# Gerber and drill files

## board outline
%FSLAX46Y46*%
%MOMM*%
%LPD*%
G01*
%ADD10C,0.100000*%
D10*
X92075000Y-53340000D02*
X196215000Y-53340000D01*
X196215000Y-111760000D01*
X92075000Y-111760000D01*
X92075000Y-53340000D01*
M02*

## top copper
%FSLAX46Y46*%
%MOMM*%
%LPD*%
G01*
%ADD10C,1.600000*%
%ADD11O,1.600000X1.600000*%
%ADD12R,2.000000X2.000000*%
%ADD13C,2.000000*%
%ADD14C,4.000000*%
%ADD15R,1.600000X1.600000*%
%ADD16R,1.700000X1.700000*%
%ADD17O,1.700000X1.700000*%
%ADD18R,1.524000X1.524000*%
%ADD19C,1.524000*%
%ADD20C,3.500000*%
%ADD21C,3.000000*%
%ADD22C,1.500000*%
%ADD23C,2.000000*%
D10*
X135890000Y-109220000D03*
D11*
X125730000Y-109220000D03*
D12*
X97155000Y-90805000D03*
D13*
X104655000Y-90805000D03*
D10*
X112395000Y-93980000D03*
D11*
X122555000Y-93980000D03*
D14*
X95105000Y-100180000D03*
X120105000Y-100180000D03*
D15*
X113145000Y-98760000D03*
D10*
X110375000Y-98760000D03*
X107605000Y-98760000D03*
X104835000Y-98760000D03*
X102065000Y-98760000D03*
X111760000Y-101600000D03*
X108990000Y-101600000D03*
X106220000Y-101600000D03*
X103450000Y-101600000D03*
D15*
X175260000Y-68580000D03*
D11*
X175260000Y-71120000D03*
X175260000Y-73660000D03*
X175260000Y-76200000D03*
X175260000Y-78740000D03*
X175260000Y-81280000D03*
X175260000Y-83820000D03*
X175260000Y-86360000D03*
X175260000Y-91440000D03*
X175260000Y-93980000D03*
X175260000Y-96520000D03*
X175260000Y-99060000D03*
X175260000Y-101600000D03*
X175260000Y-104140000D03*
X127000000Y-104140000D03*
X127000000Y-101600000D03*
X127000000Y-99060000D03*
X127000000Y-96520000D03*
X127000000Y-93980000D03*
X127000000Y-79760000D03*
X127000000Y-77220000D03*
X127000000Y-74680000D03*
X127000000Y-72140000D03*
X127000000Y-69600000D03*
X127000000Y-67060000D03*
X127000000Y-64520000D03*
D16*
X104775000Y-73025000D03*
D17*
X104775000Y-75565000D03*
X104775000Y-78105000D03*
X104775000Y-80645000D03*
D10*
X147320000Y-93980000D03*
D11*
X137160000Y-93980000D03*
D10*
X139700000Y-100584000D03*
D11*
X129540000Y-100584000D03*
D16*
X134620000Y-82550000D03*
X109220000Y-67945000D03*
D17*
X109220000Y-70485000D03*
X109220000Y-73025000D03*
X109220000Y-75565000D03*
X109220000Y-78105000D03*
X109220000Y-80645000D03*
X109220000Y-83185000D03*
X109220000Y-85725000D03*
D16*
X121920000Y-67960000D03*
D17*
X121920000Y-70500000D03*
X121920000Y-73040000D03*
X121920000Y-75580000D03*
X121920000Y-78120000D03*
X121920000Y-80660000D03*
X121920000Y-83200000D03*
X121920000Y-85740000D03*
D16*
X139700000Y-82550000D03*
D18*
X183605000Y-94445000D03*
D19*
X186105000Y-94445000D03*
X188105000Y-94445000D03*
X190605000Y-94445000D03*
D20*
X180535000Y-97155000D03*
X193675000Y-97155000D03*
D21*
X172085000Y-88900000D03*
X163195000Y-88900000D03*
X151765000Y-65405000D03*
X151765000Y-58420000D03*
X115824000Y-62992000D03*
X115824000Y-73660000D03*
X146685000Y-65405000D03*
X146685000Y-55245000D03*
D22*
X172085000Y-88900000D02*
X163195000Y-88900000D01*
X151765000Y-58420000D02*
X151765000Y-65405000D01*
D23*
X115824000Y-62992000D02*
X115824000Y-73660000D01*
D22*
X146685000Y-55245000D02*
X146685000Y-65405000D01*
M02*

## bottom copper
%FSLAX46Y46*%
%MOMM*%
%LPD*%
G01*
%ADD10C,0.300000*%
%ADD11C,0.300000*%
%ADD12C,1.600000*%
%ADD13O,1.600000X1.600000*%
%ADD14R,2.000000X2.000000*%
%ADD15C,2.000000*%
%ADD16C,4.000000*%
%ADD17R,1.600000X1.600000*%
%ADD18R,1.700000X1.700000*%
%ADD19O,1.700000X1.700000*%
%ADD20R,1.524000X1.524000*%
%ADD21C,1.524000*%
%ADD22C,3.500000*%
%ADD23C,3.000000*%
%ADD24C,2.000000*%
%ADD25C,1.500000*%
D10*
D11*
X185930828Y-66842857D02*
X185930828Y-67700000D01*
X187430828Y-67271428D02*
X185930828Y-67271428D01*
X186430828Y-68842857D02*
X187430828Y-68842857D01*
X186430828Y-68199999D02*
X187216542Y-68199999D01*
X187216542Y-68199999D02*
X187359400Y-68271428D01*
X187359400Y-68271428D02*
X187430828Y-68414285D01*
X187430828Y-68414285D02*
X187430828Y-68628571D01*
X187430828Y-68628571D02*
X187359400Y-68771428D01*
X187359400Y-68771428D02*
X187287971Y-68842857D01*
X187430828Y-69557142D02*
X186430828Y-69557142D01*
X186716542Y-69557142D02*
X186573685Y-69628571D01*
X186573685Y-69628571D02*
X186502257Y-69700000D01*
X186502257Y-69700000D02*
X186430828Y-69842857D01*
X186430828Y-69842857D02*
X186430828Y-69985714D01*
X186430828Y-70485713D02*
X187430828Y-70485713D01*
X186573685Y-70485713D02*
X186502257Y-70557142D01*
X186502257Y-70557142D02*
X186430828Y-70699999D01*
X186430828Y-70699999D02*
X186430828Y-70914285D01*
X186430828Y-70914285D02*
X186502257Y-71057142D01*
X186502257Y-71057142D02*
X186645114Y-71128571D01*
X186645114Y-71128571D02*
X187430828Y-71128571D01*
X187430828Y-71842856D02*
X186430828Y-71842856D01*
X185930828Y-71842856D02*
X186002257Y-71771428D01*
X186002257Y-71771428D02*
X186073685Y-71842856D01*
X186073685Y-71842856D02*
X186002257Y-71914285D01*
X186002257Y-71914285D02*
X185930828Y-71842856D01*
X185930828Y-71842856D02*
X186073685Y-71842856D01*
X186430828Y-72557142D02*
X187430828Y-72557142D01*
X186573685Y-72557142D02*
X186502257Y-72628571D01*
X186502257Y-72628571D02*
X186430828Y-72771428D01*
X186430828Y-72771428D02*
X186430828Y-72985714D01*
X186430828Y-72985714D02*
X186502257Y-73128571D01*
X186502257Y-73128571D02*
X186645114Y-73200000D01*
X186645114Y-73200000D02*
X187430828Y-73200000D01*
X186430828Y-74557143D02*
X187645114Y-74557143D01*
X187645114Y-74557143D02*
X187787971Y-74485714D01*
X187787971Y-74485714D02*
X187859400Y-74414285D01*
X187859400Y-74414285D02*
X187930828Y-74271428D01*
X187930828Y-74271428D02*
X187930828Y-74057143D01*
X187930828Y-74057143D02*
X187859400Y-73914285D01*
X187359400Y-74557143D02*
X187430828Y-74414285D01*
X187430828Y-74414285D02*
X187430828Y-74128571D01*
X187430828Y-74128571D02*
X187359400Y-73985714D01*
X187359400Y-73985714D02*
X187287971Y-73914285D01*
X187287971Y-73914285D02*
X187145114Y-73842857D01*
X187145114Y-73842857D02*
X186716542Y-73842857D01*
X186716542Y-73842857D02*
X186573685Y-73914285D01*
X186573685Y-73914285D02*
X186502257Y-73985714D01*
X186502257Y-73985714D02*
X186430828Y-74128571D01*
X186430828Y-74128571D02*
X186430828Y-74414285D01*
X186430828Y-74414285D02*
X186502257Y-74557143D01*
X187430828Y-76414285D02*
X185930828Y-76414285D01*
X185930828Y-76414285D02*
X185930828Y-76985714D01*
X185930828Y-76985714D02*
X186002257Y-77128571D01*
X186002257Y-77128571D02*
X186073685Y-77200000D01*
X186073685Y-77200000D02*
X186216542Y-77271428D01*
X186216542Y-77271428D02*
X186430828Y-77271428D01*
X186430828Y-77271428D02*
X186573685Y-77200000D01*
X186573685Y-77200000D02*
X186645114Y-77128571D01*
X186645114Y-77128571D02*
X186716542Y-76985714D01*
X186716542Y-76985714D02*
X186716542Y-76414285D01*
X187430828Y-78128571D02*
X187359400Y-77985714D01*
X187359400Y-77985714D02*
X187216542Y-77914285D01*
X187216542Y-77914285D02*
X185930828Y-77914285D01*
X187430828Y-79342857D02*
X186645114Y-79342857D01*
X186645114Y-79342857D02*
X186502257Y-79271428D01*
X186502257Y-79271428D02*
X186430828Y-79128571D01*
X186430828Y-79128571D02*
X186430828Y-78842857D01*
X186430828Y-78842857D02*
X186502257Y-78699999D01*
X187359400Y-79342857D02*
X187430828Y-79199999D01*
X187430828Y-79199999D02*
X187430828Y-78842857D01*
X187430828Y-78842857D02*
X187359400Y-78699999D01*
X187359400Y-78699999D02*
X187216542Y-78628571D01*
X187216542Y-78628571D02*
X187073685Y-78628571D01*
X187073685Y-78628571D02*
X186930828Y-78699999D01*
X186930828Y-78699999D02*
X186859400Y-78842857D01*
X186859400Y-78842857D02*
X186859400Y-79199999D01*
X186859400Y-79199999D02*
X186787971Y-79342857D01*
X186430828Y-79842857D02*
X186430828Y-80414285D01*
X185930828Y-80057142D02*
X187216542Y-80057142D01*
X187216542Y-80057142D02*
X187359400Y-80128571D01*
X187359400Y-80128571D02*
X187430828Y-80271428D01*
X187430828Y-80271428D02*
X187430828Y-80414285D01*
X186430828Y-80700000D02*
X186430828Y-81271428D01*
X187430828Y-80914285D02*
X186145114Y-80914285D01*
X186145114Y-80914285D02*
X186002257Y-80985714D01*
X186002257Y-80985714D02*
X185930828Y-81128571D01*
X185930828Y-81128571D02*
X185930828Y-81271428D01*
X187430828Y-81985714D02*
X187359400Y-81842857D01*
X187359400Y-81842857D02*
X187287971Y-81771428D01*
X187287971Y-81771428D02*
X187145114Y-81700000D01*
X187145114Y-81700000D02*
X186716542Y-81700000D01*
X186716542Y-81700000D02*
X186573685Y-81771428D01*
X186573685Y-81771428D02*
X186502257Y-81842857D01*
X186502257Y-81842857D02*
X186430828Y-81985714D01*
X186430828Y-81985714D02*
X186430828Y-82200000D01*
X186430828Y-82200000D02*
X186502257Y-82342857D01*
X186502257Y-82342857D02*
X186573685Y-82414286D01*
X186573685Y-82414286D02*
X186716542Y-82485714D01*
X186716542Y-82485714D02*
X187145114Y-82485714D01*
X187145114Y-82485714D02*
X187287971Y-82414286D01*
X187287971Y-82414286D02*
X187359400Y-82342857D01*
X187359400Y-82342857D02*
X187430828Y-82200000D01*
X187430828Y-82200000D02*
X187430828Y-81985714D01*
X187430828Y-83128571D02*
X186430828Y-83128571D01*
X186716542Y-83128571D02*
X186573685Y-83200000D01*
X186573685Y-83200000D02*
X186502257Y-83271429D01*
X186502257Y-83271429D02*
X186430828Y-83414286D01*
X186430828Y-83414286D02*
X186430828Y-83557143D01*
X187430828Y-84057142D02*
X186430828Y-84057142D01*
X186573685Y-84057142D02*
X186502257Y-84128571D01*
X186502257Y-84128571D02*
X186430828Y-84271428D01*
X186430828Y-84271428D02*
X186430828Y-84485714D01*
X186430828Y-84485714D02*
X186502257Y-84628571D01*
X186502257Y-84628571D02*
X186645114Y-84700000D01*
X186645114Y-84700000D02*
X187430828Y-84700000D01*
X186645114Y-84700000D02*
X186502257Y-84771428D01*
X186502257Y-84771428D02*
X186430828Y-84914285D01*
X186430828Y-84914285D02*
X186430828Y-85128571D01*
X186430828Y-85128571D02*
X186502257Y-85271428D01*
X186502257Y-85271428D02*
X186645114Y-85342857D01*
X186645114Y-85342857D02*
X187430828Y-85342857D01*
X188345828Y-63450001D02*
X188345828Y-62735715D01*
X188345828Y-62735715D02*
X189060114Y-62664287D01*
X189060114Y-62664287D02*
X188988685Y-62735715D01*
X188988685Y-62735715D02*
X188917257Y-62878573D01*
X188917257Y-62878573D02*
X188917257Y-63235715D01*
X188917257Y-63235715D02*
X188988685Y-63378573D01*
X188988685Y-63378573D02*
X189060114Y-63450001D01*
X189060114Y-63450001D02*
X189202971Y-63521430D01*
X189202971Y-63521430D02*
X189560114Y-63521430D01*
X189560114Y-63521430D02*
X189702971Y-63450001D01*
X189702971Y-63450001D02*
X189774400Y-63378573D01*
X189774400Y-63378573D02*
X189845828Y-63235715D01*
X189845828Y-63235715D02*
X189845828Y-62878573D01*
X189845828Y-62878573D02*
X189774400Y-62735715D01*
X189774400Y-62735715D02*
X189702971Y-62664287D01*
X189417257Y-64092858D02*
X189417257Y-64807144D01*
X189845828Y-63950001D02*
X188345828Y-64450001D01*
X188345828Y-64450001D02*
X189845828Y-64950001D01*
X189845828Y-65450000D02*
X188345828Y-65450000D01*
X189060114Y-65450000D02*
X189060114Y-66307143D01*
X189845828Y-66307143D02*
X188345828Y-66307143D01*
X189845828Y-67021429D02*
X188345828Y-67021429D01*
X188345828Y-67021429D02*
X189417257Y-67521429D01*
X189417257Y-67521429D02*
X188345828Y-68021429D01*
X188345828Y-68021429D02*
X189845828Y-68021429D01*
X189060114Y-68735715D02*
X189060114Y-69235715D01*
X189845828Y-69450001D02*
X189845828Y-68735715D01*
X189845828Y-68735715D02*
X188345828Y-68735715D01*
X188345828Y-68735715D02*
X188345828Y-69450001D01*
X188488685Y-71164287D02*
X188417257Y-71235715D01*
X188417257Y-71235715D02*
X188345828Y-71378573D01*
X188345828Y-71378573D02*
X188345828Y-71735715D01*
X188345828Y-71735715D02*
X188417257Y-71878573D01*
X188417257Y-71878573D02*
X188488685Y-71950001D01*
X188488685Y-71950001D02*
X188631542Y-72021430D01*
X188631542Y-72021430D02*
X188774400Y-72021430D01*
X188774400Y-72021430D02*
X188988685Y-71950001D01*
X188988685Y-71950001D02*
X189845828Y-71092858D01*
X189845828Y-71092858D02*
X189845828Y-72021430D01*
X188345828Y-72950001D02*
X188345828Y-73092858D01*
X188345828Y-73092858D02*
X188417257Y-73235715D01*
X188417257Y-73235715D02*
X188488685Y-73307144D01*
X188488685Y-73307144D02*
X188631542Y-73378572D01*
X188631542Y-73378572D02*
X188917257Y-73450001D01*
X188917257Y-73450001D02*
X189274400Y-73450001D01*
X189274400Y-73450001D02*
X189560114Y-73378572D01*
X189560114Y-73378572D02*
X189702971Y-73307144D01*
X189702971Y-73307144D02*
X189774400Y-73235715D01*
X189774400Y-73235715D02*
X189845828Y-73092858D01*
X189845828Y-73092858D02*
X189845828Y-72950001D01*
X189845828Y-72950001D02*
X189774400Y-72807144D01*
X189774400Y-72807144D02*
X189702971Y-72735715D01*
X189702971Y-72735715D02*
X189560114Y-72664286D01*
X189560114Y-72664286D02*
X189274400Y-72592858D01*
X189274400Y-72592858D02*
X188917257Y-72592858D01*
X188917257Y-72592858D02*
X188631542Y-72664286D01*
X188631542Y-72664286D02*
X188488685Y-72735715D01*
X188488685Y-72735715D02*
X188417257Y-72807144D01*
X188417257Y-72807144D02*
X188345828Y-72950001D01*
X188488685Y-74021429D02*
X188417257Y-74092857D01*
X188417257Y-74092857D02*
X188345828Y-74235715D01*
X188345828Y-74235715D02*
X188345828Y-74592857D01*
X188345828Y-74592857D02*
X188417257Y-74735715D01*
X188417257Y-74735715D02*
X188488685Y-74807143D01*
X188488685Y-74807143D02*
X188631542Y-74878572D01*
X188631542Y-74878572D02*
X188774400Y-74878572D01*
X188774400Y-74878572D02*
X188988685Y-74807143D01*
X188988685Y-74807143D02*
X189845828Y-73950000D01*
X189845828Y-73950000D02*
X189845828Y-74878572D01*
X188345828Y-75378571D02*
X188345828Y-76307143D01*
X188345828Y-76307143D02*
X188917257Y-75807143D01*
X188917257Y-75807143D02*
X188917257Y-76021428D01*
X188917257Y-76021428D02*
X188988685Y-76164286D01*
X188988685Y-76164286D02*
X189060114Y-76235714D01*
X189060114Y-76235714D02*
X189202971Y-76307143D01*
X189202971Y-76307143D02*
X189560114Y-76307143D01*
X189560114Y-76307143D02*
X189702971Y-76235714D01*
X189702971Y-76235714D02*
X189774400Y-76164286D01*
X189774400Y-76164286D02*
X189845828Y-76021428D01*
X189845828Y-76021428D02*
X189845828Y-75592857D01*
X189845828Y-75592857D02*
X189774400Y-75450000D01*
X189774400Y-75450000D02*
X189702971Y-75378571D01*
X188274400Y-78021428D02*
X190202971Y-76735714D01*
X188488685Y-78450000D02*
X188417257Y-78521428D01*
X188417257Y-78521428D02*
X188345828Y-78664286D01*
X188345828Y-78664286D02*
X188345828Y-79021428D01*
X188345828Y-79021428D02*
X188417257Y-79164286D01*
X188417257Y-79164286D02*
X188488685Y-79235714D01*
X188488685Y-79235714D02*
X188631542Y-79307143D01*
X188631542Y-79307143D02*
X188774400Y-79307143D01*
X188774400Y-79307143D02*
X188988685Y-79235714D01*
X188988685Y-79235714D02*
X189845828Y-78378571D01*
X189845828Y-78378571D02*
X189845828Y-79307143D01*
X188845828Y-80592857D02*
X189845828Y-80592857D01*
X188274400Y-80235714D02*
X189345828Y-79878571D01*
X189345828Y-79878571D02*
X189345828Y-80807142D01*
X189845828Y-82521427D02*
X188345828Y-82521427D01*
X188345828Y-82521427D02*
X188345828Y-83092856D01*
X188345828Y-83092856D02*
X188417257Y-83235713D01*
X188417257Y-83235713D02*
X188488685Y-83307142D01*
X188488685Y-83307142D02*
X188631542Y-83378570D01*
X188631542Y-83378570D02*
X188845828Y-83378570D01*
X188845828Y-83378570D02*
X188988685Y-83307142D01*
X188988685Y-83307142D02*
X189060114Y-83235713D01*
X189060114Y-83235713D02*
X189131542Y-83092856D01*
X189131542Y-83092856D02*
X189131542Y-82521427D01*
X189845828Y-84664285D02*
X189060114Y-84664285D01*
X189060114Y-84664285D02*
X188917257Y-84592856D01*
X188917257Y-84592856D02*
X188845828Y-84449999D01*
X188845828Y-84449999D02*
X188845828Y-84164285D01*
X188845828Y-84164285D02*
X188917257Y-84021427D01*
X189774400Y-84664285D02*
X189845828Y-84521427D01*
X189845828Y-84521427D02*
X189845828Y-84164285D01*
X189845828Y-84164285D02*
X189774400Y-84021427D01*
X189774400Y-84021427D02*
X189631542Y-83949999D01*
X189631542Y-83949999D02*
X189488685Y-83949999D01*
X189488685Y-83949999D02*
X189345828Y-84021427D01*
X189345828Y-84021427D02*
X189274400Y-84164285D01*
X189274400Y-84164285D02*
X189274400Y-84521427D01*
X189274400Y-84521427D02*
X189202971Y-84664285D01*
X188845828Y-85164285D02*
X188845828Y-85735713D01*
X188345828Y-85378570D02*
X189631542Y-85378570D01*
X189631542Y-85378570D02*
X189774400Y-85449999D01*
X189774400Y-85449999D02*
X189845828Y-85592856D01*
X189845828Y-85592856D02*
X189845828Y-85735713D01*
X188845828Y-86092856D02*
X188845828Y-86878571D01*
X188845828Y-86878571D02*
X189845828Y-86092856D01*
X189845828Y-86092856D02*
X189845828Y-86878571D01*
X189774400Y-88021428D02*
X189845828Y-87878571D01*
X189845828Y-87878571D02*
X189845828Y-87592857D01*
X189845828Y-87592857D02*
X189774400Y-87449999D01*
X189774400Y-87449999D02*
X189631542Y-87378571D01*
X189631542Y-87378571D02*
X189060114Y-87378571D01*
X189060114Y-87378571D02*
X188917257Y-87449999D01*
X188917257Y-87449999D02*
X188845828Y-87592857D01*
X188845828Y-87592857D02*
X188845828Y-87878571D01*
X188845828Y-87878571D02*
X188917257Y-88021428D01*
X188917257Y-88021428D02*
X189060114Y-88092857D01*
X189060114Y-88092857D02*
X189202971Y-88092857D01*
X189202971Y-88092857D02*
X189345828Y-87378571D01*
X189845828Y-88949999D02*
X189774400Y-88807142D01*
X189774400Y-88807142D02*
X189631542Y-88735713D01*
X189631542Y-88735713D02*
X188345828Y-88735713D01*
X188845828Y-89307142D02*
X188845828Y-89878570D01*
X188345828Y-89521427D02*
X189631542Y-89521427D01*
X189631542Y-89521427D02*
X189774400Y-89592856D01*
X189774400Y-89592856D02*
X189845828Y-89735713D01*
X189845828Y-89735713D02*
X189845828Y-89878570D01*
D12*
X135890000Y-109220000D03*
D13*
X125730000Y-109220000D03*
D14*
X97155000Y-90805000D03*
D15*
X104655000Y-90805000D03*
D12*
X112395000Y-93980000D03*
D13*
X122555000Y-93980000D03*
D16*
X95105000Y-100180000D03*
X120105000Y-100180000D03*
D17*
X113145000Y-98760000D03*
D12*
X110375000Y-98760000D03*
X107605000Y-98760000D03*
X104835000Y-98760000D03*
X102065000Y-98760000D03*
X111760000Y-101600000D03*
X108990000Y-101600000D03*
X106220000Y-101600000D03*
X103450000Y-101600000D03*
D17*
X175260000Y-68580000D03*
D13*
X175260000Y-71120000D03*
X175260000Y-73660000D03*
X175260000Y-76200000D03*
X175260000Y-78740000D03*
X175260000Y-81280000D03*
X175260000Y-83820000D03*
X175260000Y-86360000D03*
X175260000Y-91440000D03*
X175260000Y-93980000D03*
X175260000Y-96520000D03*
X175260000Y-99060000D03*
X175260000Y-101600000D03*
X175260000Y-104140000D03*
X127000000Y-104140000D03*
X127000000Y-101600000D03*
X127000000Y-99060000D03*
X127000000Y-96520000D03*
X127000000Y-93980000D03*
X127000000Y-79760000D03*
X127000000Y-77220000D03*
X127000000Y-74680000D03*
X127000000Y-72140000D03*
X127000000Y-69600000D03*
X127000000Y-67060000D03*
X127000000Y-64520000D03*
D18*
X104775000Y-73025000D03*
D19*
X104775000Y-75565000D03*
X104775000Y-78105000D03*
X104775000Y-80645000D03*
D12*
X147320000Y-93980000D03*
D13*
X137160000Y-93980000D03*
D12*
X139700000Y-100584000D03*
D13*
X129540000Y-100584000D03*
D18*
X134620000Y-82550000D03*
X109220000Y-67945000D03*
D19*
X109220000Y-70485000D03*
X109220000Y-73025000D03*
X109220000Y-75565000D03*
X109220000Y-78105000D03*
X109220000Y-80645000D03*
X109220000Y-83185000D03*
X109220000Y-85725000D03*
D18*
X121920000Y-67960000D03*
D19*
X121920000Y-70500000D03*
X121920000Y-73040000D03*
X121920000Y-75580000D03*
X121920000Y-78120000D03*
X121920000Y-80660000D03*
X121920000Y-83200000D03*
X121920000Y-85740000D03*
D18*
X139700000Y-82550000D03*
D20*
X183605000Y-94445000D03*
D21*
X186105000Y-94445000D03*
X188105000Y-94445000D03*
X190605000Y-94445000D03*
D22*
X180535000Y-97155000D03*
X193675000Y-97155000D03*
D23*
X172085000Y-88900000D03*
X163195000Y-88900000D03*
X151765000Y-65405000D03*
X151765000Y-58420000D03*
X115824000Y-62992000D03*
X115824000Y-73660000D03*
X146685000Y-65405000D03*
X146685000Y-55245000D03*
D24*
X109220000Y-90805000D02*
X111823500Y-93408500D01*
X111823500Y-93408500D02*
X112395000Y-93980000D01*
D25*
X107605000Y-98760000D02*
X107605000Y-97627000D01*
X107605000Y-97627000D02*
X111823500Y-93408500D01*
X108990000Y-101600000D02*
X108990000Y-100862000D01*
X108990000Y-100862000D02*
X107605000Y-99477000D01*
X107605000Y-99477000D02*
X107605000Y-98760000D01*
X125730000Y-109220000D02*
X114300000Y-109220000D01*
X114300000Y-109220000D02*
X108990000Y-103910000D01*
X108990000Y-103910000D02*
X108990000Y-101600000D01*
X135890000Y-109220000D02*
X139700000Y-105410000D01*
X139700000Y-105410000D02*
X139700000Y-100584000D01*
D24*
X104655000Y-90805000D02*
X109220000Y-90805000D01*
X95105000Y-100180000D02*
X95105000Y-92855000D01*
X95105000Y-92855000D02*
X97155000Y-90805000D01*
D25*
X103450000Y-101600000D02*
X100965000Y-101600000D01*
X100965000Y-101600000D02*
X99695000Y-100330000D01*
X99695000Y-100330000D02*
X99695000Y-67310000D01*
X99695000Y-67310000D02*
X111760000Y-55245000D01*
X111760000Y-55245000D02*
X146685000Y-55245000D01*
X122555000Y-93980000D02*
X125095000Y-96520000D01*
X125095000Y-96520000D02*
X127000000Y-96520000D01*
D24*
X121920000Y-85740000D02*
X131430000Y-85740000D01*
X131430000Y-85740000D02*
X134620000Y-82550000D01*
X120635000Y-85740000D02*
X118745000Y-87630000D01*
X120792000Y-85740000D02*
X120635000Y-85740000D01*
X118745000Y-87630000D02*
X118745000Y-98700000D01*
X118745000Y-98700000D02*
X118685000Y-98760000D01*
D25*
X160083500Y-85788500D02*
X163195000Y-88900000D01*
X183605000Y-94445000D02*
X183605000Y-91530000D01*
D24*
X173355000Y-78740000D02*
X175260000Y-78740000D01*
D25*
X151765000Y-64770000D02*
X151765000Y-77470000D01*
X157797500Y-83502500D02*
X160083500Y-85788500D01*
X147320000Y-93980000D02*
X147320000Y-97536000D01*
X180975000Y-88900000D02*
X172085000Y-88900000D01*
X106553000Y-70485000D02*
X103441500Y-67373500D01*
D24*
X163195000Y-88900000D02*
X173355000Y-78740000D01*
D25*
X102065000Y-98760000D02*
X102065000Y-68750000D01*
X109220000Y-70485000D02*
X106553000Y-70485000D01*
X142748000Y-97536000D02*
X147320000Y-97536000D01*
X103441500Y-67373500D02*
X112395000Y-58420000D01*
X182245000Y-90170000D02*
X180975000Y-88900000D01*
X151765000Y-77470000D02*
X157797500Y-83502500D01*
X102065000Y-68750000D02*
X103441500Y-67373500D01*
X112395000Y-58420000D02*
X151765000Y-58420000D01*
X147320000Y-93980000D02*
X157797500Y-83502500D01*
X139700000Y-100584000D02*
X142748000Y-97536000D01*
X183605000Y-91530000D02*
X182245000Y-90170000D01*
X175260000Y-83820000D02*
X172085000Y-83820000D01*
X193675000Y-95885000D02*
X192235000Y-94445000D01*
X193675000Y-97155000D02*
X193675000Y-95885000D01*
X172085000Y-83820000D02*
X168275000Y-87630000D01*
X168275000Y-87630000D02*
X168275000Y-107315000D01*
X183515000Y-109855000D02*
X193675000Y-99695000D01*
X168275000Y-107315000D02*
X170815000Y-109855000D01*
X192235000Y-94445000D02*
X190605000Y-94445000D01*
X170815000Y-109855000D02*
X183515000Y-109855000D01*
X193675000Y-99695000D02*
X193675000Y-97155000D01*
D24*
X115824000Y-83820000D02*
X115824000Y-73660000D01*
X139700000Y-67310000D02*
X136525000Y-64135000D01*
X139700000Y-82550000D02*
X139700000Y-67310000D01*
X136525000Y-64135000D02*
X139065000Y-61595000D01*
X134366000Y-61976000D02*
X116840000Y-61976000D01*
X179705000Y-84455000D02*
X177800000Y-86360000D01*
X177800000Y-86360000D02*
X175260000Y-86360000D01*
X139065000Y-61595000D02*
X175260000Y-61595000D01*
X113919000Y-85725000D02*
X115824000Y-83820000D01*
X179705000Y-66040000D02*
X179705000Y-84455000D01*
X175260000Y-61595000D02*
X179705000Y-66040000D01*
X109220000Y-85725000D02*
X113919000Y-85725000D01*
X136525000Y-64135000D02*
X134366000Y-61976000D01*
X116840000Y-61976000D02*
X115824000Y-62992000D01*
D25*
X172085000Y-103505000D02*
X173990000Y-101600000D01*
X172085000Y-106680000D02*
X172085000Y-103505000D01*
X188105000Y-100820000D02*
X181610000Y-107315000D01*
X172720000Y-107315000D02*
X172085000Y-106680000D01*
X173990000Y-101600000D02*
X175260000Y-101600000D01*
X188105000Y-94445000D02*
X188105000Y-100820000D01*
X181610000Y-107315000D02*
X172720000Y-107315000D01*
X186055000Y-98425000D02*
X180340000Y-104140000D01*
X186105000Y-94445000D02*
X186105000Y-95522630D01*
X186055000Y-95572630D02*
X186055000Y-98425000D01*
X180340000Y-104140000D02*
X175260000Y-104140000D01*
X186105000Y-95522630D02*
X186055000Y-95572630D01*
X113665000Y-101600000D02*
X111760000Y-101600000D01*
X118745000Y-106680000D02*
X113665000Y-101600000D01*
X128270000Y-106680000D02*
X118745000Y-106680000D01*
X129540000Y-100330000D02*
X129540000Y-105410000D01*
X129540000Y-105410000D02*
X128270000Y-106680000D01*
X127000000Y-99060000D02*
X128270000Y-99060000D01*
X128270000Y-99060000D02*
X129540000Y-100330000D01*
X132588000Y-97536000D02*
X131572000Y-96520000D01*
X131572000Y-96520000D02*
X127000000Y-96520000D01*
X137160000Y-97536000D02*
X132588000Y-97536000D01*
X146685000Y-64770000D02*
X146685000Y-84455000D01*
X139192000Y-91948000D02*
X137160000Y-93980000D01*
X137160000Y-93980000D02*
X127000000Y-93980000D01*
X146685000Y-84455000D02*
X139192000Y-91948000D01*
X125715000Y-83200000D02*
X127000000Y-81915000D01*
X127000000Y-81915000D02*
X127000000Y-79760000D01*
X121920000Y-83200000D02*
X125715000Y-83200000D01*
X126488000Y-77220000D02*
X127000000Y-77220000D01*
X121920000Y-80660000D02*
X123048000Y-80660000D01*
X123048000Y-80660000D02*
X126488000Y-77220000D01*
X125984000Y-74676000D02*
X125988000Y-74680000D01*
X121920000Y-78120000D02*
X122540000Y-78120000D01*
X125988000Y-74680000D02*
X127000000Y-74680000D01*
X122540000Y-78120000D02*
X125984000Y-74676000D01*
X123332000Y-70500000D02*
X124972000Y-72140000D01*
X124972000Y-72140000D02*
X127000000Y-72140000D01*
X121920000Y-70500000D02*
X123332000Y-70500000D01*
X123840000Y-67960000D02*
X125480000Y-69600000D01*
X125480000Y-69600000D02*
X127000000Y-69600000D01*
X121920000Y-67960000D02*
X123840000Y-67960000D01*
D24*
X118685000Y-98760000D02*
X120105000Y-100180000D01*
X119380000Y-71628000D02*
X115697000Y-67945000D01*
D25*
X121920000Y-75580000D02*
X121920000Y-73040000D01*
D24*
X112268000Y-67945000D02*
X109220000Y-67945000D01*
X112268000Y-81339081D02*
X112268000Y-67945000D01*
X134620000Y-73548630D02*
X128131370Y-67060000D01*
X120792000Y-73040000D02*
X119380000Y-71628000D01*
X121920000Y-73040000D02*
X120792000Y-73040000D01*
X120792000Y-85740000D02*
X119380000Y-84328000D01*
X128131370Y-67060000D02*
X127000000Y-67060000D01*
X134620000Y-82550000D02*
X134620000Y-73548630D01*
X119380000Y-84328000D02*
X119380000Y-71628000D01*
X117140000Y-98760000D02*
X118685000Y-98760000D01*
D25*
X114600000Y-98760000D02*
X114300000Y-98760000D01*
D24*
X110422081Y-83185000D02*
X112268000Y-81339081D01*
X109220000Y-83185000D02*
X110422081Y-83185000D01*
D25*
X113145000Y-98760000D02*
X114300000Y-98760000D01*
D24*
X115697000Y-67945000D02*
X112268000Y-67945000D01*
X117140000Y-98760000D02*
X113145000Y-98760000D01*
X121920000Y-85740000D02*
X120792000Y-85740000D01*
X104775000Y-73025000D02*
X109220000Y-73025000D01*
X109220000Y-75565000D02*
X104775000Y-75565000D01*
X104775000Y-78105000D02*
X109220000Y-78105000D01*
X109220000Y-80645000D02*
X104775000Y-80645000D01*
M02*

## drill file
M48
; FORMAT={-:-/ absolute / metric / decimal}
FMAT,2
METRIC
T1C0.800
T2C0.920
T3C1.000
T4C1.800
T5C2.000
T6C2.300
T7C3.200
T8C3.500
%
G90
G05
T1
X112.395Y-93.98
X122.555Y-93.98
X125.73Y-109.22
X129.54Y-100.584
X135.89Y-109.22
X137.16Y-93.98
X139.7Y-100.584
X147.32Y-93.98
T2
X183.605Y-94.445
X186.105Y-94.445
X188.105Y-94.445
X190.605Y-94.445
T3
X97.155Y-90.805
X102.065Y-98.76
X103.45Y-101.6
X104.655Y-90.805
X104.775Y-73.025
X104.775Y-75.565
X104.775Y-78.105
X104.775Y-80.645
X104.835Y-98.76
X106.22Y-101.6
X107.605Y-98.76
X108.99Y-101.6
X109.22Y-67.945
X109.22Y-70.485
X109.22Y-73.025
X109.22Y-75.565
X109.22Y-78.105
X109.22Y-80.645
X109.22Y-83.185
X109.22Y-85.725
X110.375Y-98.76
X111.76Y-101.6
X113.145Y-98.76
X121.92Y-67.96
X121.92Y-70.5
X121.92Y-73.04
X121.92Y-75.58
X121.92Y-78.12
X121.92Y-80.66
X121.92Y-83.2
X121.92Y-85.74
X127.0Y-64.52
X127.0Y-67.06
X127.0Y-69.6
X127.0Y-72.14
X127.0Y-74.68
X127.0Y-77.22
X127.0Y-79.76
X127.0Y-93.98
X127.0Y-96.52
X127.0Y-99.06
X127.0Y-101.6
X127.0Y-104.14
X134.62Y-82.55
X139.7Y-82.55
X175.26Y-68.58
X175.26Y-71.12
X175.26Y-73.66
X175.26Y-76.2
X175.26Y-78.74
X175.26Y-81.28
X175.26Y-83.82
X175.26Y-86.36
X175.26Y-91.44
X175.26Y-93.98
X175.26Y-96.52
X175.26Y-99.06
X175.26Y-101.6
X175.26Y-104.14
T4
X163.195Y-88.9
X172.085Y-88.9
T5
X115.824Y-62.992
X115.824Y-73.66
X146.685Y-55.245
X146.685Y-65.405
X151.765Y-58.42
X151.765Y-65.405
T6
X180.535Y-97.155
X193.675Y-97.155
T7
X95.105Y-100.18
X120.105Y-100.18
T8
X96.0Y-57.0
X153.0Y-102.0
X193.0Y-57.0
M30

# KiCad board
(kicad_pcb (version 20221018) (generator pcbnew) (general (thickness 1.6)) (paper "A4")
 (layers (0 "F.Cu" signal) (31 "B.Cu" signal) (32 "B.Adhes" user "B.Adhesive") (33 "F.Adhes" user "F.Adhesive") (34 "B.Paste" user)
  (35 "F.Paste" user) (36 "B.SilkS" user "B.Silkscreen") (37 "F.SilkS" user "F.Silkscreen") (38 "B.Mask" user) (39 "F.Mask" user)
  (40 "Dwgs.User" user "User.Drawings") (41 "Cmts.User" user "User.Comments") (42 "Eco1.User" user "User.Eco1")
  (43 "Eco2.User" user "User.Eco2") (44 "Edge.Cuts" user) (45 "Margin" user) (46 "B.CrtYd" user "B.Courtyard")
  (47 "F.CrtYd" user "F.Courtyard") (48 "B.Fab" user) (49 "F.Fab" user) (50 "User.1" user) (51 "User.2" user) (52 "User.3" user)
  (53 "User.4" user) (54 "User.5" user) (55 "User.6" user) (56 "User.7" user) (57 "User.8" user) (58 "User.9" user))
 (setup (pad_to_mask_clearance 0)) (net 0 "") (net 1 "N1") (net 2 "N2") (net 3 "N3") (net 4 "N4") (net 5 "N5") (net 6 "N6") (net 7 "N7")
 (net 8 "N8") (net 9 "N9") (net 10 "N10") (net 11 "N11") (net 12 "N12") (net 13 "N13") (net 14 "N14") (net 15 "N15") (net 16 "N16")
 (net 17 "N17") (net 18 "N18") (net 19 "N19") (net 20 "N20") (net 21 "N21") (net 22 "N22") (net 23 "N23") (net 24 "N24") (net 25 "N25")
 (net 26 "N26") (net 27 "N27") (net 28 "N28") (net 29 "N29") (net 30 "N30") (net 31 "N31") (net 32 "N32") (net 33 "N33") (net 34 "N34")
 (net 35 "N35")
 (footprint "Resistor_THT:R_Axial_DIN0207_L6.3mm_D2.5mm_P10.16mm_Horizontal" (layer "F.Cu") (at 135.89 109.22 180)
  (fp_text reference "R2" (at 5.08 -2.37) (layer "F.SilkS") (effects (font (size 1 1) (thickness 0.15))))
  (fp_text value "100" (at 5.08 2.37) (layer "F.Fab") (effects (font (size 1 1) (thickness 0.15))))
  (pad "1" thru_hole circle (at 0 0 180) (size 1.6 1.6) (drill 0.8) (layers "*.Cu" "*.Mask") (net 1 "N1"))
  (pad "2" thru_hole oval (at 10.16 0 180) (size 1.6 1.6) (drill 0.8) (layers "*.Cu" "*.Mask") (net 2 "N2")))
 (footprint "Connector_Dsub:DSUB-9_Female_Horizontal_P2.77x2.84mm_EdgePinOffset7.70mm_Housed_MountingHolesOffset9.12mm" (layer "F.Cu")
  (at 113.145 98.76)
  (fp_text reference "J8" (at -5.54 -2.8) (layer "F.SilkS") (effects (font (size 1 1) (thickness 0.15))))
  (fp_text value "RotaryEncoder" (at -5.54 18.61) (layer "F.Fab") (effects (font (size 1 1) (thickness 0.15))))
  (pad "0" thru_hole circle (at -18.04 1.42) (size 4 4) (drill 3.2) (layers "*.Cu" "*.Mask") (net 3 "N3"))
  (pad "0" thru_hole circle (at 6.96 1.42) (size 4 4) (drill 3.2) (layers "*.Cu" "*.Mask") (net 3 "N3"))
  (pad "1" thru_hole rect (at 0 0) (size 1.6 1.6) (drill 1) (layers "*.Cu" "*.Mask") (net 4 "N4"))
  (pad "2" thru_hole circle (at -2.77 0) (size 1.6 1.6) (drill 1) (layers "*.Cu" "*.Mask") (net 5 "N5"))
  (pad "3" thru_hole circle (at -5.54 0) (size 1.6 1.6) (drill 1) (layers "*.Cu" "*.Mask") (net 2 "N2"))
  (pad "4" thru_hole circle (at -8.31 0) (size 1.6 1.6) (drill 1) (layers "*.Cu" "*.Mask") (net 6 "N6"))
  (pad "5" thru_hole circle (at -11.08 0) (size 1.6 1.6) (drill 1) (layers "*.Cu" "*.Mask") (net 1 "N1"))
  (pad "6" thru_hole circle (at -1.385 2.84) (size 1.6 1.6) (drill 1) (layers "*.Cu" "*.Mask") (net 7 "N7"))
  (pad "7" thru_hole circle (at -4.155 2.84) (size 1.6 1.6) (drill 1) (layers "*.Cu" "*.Mask") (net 2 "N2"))
  (pad "8" thru_hole circle (at -6.925 2.84) (size 1.6 1.6) (drill 1) (layers "*.Cu" "*.Mask") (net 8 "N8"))
  (pad "9" thru_hole circle (at -9.695 2.84) (size 1.6 1.6) (drill 1) (layers "*.Cu" "*.Mask") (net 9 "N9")))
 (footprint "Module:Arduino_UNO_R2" (layer "F.Cu") (at 175.26 68.58 -90)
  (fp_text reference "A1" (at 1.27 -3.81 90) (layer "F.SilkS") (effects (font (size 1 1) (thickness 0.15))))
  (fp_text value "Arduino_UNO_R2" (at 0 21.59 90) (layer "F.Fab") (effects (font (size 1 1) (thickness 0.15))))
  (pad "1" thru_hole rect (at 0 0) (size 1.6 1.6) (drill 1) (layers "*.Cu" "*.Mask") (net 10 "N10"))
  (pad "2" thru_hole oval (at 2.54 0) (size 1.6 1.6) (drill 1) (layers "*.Cu" "*.Mask") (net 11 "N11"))
  (pad "3" thru_hole oval (at 5.08 0) (size 1.6 1.6) (drill 1) (layers "*.Cu" "*.Mask") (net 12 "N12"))
  (pad "4" thru_hole oval (at 7.62 0) (size 1.6 1.6) (drill 1) (layers "*.Cu" "*.Mask") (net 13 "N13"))
  (pad "5" thru_hole oval (at 10.16 0) (size 1.6 1.6) (drill 1) (layers "*.Cu" "*.Mask") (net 1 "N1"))
  (pad "6" thru_hole oval (at 12.7 0) (size 1.6 1.6) (drill 1) (layers "*.Cu" "*.Mask") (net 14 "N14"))
  (pad "7" thru_hole oval (at 15.24 0) (size 1.6 1.6) (drill 1) (layers "*.Cu" "*.Mask") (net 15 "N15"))
  (pad "8" thru_hole oval (at 17.78 0) (size 1.6 1.6) (drill 1) (layers "*.Cu" "*.Mask") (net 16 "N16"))
  (pad "9" thru_hole oval (at 22.86 0) (size 1.6 1.6) (drill 1) (layers "*.Cu" "*.Mask") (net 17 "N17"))
  (pad "10" thru_hole oval (at 25.4 0) (size 1.6 1.6) (drill 1) (layers "*.Cu" "*.Mask") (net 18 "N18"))
  (pad "11" thru_hole oval (at 27.94 0) (size 1.6 1.6) (drill 1) (layers "*.Cu" "*.Mask") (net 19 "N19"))
  (pad "12" thru_hole oval (at 30.48 0) (size 1.6 1.6) (drill 1) (layers "*.Cu" "*.Mask") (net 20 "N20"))
  (pad "13" thru_hole oval (at 33.02 0) (size 1.6 1.6) (drill 1) (layers "*.Cu" "*.Mask") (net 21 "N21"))
  (pad "14" thru_hole oval (at 35.56 0) (size 1.6 1.6) (drill 1) (layers "*.Cu" "*.Mask") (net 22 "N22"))
  (pad "15" thru_hole oval (at 35.56 48.26) (size 1.6 1.6) (drill 1) (layers "*.Cu" "*.Mask") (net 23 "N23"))
  (pad "16" thru_hole oval (at 33.02 48.26) (size 1.6 1.6) (drill 1) (layers "*.Cu" "*.Mask") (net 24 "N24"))
  (pad "17" thru_hole oval (at 30.48 48.26) (size 1.6 1.6) (drill 1) (layers "*.Cu" "*.Mask") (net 7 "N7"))
  (pad "18" thru_hole oval (at 27.94 48.26) (size 1.6 1.6) (drill 1) (layers "*.Cu" "*.Mask") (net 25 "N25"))
  (pad "19" thru_hole oval (at 25.4 48.26) (size 1.6 1.6) (drill 1) (layers "*.Cu" "*.Mask") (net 9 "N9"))
  (pad "24" thru_hole oval (at 11.18 48.26) (size 1.6 1.6) (drill 1) (layers "*.Cu" "*.Mask") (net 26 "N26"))
  (pad "25" thru_hole oval (at 8.64 48.26) (size 1.6 1.6) (drill 1) (layers "*.Cu" "*.Mask") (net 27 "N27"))
  (pad "26" thru_hole oval (at 6.1 48.26) (size 1.6 1.6) (drill 1) (layers "*.Cu" "*.Mask") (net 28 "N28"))
  (pad "27" thru_hole oval (at 3.56 48.26) (size 1.6 1.6) (drill 1) (layers "*.Cu" "*.Mask") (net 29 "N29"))
  (pad "28" thru_hole oval (at 1.02 48.26) (size 1.6 1.6) (drill 1) (layers "*.Cu" "*.Mask") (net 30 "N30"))
  (pad "29" thru_hole oval (at -1.52 48.26) (size 1.6 1.6) (drill 1) (layers "*.Cu" "*.Mask") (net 4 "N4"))
  (pad "30" thru_hole oval (at -4.06 48.26) (size 1.6 1.6) (drill 1) (layers "*.Cu" "*.Mask") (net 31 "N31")))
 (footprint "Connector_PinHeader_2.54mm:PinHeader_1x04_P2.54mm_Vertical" (layer "F.Cu") (at 104.775 73.025)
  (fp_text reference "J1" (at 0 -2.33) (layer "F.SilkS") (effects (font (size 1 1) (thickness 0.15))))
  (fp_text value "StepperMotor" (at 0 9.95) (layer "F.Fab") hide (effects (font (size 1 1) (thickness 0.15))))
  (pad "1" thru_hole rect (at 0 0) (size 1.7 1.7) (drill 1) (layers "*.Cu" "*.Mask") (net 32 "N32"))
  (pad "2" thru_hole oval (at 0 2.54) (size 1.7 1.7) (drill 1) (layers "*.Cu" "*.Mask") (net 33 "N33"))
  (pad "3" thru_hole oval (at 0 5.08) (size 1.7 1.7) (drill 1) (layers "*.Cu" "*.Mask") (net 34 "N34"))
  (pad "4" thru_hole oval (at 0 7.62) (size 1.7 1.7) (drill 1) (layers "*.Cu" "*.Mask") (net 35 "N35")))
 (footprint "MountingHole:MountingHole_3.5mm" (layer "F.Cu") (at 193 57)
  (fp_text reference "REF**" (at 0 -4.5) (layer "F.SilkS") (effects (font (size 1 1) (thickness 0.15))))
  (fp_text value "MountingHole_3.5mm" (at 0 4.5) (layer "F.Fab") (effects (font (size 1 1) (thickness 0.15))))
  (pad "" np_thru_hole circle (at 0 0) (size 3.5 3.5) (drill 3.5) (layers "*.Cu" "*.Mask")))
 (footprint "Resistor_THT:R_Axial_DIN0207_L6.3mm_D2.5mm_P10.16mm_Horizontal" (layer "F.Cu") (at 147.32 93.98 180)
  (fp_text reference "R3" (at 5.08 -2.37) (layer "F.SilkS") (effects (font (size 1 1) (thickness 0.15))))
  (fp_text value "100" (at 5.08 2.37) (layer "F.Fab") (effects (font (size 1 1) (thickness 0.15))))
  (pad "1" thru_hole circle (at 0 0 180) (size 1.6 1.6) (drill 0.8) (layers "*.Cu" "*.Mask") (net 1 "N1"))
  (pad "2" thru_hole oval (at 10.16 0 180) (size 1.6 1.6) (drill 0.8) (layers "*.Cu" "*.Mask") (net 9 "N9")))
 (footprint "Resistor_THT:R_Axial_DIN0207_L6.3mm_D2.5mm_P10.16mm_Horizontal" (layer "F.Cu") (at 139.7 100.584 180)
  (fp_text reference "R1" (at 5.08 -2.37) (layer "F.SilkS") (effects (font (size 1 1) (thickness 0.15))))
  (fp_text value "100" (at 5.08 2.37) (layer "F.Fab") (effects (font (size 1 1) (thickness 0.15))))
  (pad "1" thru_hole circle (at 0 0 180) (size 1.6 1.6) (drill 0.8) (layers "*.Cu" "*.Mask") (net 1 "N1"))
  (pad "2" thru_hole oval (at 10.16 0 180) (size 1.6 1.6) (drill 0.8) (layers "*.Cu" "*.Mask") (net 7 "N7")))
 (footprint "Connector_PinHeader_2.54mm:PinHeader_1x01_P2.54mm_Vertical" (layer "F.Cu") (at 134.62 82.55)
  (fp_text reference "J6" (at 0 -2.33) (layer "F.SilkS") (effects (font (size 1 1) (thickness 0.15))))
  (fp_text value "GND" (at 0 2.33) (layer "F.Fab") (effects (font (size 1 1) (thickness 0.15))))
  (pad "1" thru_hole rect (at 0 0) (size 1.7 1.7) (drill 1) (layers "*.Cu" "*.Mask") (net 4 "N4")))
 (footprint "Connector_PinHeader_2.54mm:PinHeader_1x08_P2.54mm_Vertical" (layer "F.Cu") (at 109.22 67.945)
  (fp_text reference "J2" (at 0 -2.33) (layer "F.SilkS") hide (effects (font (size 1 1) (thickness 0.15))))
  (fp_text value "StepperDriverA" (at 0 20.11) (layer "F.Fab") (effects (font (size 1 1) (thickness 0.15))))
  (pad "1" thru_hole rect (at 0 0) (size 1.7 1.7) (drill 1) (layers "*.Cu" "*.Mask") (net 4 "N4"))
  (pad "2" thru_hole oval (at 0 2.54) (size 1.7 1.7) (drill 1) (layers "*.Cu" "*.Mask") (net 1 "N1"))
  (pad "3" thru_hole oval (at 0 5.08) (size 1.7 1.7) (drill 1) (layers "*.Cu" "*.Mask") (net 32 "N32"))
  (pad "4" thru_hole oval (at 0 7.62) (size 1.7 1.7) (drill 1) (layers "*.Cu" "*.Mask") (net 33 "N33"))
  (pad "5" thru_hole oval (at 0 10.16) (size 1.7 1.7) (drill 1) (layers "*.Cu" "*.Mask") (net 34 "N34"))
  (pad "6" thru_hole oval (at 0 12.7) (size 1.7 1.7) (drill 1) (layers "*.Cu" "*.Mask") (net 35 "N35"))
  (pad "7" thru_hole oval (at 0 15.24) (size 1.7 1.7) (drill 1) (layers "*.Cu" "*.Mask") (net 4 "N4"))
  (pad "8" thru_hole oval (at 0 17.78) (size 1.7 1.7) (drill 1) (layers "*.Cu" "*.Mask") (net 16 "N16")))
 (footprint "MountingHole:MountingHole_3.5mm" (layer "F.Cu") (at 153 102)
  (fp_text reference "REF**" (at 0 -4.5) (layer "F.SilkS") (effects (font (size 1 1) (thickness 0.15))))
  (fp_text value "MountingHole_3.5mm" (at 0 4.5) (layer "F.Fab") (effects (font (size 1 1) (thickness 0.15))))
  (pad "" np_thru_hole circle (at 0 0) (size 3.5 3.5) (drill 3.5) (layers "*.Cu" "*.Mask")))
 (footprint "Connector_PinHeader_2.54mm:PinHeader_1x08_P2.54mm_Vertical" (layer "F.Cu") (at 121.92 67.96)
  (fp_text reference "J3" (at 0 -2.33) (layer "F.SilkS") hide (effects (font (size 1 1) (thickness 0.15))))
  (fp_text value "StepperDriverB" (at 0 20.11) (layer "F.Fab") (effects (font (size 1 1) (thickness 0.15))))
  (pad "1" thru_hole rect (at 0 0) (size 1.7 1.7) (drill 1) (layers "*.Cu" "*.Mask") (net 30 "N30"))
  (pad "2" thru_hole oval (at 0 2.54) (size 1.7 1.7) (drill 1) (layers "*.Cu" "*.Mask") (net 29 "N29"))
  (pad "3" thru_hole oval (at 0 5.08) (size 1.7 1.7) (drill 1) (layers "*.Cu" "*.Mask") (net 4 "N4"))
  (pad "4" thru_hole oval (at 0 7.62) (size 1.7 1.7) (drill 1) (layers "*.Cu" "*.Mask") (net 4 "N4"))
  (pad "5" thru_hole oval (at 0 10.16) (size 1.7 1.7) (drill 1) (layers "*.Cu" "*.Mask") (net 28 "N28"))
  (pad "6" thru_hole oval (at 0 12.7) (size 1.7 1.7) (drill 1) (layers "*.Cu" "*.Mask") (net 27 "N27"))
  (pad "7" thru_hole oval (at 0 15.24) (size 1.7 1.7) (drill 1) (layers "*.Cu" "*.Mask") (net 26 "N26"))
  (pad "8" thru_hole oval (at 0 17.78) (size 1.7 1.7) (drill 1) (layers "*.Cu" "*.Mask") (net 4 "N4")))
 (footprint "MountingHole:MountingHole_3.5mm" (layer "F.Cu") (at 96 57)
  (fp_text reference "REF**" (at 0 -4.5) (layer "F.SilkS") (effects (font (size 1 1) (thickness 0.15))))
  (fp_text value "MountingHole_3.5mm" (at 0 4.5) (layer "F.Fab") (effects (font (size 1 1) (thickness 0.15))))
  (pad "" np_thru_hole circle (at 0 0) (size 3.5 3.5) (drill 3.5) (layers "*.Cu" "*.Mask")))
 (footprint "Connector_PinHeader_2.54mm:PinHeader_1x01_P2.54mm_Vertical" (layer "F.Cu") (at 139.7 82.55)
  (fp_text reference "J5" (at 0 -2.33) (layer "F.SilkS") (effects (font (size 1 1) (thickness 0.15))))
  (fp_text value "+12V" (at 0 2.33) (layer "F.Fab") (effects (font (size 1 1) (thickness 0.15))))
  (pad "1" thru_hole rect (at 0 0) (size 1.7 1.7) (drill 1) (layers "*.Cu" "*.Mask") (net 16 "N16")))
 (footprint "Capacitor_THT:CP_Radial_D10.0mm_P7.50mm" (layer "F.Cu") (at 97.155 90.805)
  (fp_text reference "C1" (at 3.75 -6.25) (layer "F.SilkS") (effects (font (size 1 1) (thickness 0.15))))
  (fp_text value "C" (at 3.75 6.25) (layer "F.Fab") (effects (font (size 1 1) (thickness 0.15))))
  (pad "1" thru_hole rect (at 0 0) (size 2 2) (drill 1) (layers "*.Cu" "*.Mask") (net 4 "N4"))
  (pad "2" thru_hole circle (at 7.5 0) (size 2 2) (drill 1) (layers "*.Cu" "*.Mask") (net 2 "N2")))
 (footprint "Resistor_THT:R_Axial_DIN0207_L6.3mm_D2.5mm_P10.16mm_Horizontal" (layer "F.Cu") (at 112.395 93.98)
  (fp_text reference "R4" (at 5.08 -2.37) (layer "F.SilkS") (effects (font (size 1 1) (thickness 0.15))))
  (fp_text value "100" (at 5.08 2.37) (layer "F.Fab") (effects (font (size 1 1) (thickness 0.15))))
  (pad "1" thru_hole circle (at 0 0) (size 1.6 1.6) (drill 0.8) (layers "*.Cu" "*.Mask") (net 2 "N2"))
  (pad "2" thru_hole oval (at 10.16 0) (size 1.6 1.6) (drill 0.8) (layers "*.Cu" "*.Mask") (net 25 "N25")))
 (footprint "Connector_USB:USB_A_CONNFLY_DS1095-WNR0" (layer "F.Cu") (at 183.605 94.445)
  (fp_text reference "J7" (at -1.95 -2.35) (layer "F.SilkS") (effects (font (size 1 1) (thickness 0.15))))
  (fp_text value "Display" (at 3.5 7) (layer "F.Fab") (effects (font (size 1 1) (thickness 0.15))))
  (pad "1" thru_hole rect (at 0 0) (size 1.524 1.524) (drill 0.92) (layers "*.Cu" "*.Mask") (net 1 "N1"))
  (pad "2" thru_hole circle (at 2.5 0) (size 1.524 1.524) (drill 0.92) (layers "*.Cu" "*.Mask") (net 22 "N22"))
  (pad "3" thru_hole circle (at 4.5 0) (size 1.524 1.524) (drill 0.92) (layers "*.Cu" "*.Mask") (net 21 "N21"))
  (pad "4" thru_hole circle (at 7 0) (size 1.524 1.524) (drill 0.92) (layers "*.Cu" "*.Mask") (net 15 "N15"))
  (pad "5" thru_hole circle (at -3.07 2.71) (size 3.5 3.5) (drill 2.3) (layers "*.Cu" "*.Mask") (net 15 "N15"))
  (pad "5" thru_hole circle (at 10.07 2.71) (size 3.5 3.5) (drill 2.3) (layers "*.Cu" "*.Mask") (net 15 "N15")))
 (gr_rect (start 92.075 53.34) (end 196.215 111.76) (stroke (width 0.1) (type default)) (fill none) (layer "Edge.Cuts"))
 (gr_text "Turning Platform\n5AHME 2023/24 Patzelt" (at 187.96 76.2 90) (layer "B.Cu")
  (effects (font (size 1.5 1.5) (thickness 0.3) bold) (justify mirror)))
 (segment (start 172.085 88.9) (end 163.195 88.9) (width 1.5) (layer "F.Cu") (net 1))
 (segment (start 151.765 58.42) (end 151.765 65.405) (width 1.5) (layer "F.Cu") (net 1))
 (via (at 172.085 88.9) (size 3) (drill 1.8) (layers "F.Cu" "B.Cu") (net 1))
 (via (at 163.195 88.9) (size 3) (drill 1.8) (layers "F.Cu" "B.Cu") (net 1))
 (via (at 151.765 65.405) (size 3) (drill 2) (layers "F.Cu" "B.Cu") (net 1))
 (via (at 151.765 58.42) (size 3) (drill 2) (layers "F.Cu" "B.Cu") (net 1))
 (segment (start 135.89 109.22) (end 139.7 105.41) (width 1.5) (layer "B.Cu") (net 1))
 (segment (start 160.0835 85.7885) (end 163.195 88.9) (width 1.5) (layer "B.Cu") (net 1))
 (segment (start 183.605 94.445) (end 183.605 91.53) (width 1.5) (layer "B.Cu") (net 1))
 (segment (start 173.355 78.74) (end 175.26 78.74) (width 2) (layer "B.Cu") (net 1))
 (segment (start 151.765 64.77) (end 151.765 77.47) (width 1.5) (layer "B.Cu") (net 1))
 (segment (start 157.7975 83.5025) (end 160.0835 85.7885) (width 1.5) (layer "B.Cu") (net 1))
 (segment (start 147.32 93.98) (end 147.32 97.536) (width 1.5) (layer "B.Cu") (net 1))
 (segment (start 180.975 88.9) (end 172.085 88.9) (width 1.5) (layer "B.Cu") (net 1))
 (segment (start 106.553 70.485) (end 103.4415 67.3735) (width 1.5) (layer "B.Cu") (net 1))
 (segment (start 163.195 88.9) (end 173.355 78.74) (width 2) (layer "B.Cu") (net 1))
 (segment (start 102.065 98.76) (end 102.065 68.75) (width 1.5) (layer "B.Cu") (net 1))
 (segment (start 109.22 70.485) (end 106.553 70.485) (width 1.5) (layer "B.Cu") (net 1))
 (segment (start 142.748 97.536) (end 147.32 97.536) (width 1.5) (layer "B.Cu") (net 1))
 (segment (start 103.4415 67.3735) (end 112.395 58.42) (width 1.5) (layer "B.Cu") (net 1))
 (segment (start 182.245 90.17) (end 180.975 88.9) (width 1.5) (layer "B.Cu") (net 1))
 (segment (start 151.765 77.47) (end 157.7975 83.5025) (width 1.5) (layer "B.Cu") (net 1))
 (segment (start 139.7 105.41) (end 139.7 100.584) (width 1.5) (layer "B.Cu") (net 1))
 (segment (start 102.065 68.75) (end 103.4415 67.3735) (width 1.5) (layer "B.Cu") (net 1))
 (segment (start 112.395 58.42) (end 151.765 58.42) (width 1.5) (layer "B.Cu") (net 1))
 (segment (start 147.32 93.98) (end 157.7975 83.5025) (width 1.5) (layer "B.Cu") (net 1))
 (segment (start 139.7 100.584) (end 142.748 97.536) (width 1.5) (layer "B.Cu") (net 1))
 (segment (start 183.605 91.53) (end 182.245 90.17) (width 1.5) (layer "B.Cu") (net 1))
 (segment (start 175.26 83.82) (end 172.085 83.82) (width 1.5) (layer "B.Cu") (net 15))
 (segment (start 193.675 95.885) (end 192.235 94.445) (width 1.5) (layer "B.Cu") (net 15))
 (segment (start 193.675 97.155) (end 193.675 95.885) (width 1.5) (layer "B.Cu") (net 15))
 (segment (start 172.085 83.82) (end 168.275 87.63) (width 1.5) (layer "B.Cu") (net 15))
 (segment (start 168.275 87.63) (end 168.275 107.315) (width 1.5) (layer "B.Cu") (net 15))
 (segment (start 183.515 109.855) (end 193.675 99.695) (width 1.5) (layer "B.Cu") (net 15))
 (segment (start 168.275 107.315) (end 170.815 109.855) (width 1.5) (layer "B.Cu") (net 15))
 (segment (start 192.235 94.445) (end 190.605 94.445) (width 1.5) (layer "B.Cu") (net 15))
 (segment (start 170.815 109.855) (end 183.515 109.855) (width 1.5) (layer "B.Cu") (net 15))
 (segment (start 193.675 99.695) (end 193.675 97.155) (width 1.5) (layer "B.Cu") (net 15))
 (segment (start 115.824 62.992) (end 115.824 73.66) (width 2) (layer "F.Cu") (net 16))
 (via (at 115.824 62.992) (size 3) (drill 2) (layers "F.Cu" "B.Cu") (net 16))
 (via (at 115.824 73.66) (size 3) (drill 2) (layers "F.Cu" "B.Cu") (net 16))
 (segment (start 115.824 83.82) (end 115.824 73.66) (width 2) (layer "B.Cu") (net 16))
 (segment (start 139.7 67.31) (end 136.525 64.135) (width 2) (layer "B.Cu") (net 16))
 (segment (start 139.7 82.55) (end 139.7 67.31) (width 2) (layer "B.Cu") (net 16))
 (segment (start 136.525 64.135) (end 139.065 61.595) (width 2) (layer "B.Cu") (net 16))
 (segment (start 134.366 61.976) (end 116.84 61.976) (width 2) (layer "B.Cu") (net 16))
 (segment (start 179.705 84.455) (end 177.8 86.36) (width 2) (layer "B.Cu") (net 16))
 (segment (start 177.8 86.36) (end 175.26 86.36) (width 2) (layer "B.Cu") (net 16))
 (segment (start 139.065 61.595) (end 175.26 61.595) (width 2) (layer "B.Cu") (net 16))
 (segment (start 113.919 85.725) (end 115.824 83.82) (width 2) (layer "B.Cu") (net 16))
 (segment (start 179.705 66.04) (end 179.705 84.455) (width 2) (layer "B.Cu") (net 16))
 (segment (start 175.26 61.595) (end 179.705 66.04) (width 2) (layer "B.Cu") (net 16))
 (segment (start 109.22 85.725) (end 113.919 85.725) (width 2) (layer "B.Cu") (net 16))
 (segment (start 136.525 64.135) (end 134.366 61.976) (width 2) (layer "B.Cu") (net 16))
 (segment (start 116.84 61.976) (end 115.824 62.992) (width 2) (layer "B.Cu") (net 16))
 (segment (start 172.085 103.505) (end 173.99 101.6) (width 1.5) (layer "B.Cu") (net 21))
 (segment (start 172.085 106.68) (end 172.085 103.505) (width 1.5) (layer "B.Cu") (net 21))
 (segment (start 188.105 100.82) (end 181.61 107.315) (width 1.5) (layer "B.Cu") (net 21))
 (segment (start 172.72 107.315) (end 172.085 106.68) (width 1.5) (layer "B.Cu") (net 21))
 (segment (start 173.99 101.6) (end 175.26 101.6) (width 1.5) (layer "B.Cu") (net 21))
 (segment (start 188.105 94.445) (end 188.105 100.82) (width 1.5) (layer "B.Cu") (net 21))
 (segment (start 181.61 107.315) (end 172.72 107.315) (width 1.5) (layer "B.Cu") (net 21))
 (segment (start 186.055 98.425) (end 180.34 104.14) (width 1.5) (layer "B.Cu") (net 22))
 (segment (start 186.105 94.445) (end 186.105 95.52263) (width 1.5) (layer "B.Cu") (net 22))
 (segment (start 186.055 95.57263) (end 186.055 98.425) (width 1.5) (layer "B.Cu") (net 22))
 (segment (start 180.34 104.14) (end 175.26 104.14) (width 1.5) (layer "B.Cu") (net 22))
 (segment (start 186.105 95.52263) (end 186.055 95.57263) (width 1.5) (layer "B.Cu") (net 22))
 (segment (start 113.665 101.6) (end 111.76 101.6) (width 1.5) (layer "B.Cu") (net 7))
 (segment (start 118.745 106.68) (end 113.665 101.6) (width 1.5) (layer "B.Cu") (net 7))
 (segment (start 128.27 106.68) (end 118.745 106.68) (width 1.5) (layer "B.Cu") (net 7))
 (segment (start 129.54 100.33) (end 129.54 105.41) (width 1.5) (layer "B.Cu") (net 7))
 (segment (start 129.54 105.41) (end 128.27 106.68) (width 1.5) (layer "B.Cu") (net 7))
 (segment (start 127 99.06) (end 128.27 99.06) (width 1.5) (layer "B.Cu") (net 7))
 (segment (start 128.27 99.06) (end 129.54 100.33) (width 1.5) (layer "B.Cu") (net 7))
 (segment (start 122.555 93.98) (end 125.095 96.52) (width 1.5) (layer "B.Cu") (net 25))
 (segment (start 132.588 97.536) (end 131.572 96.52) (width 1.5) (layer "B.Cu") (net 25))
 (segment (start 131.572 96.52) (end 127 96.52) (width 1.5) (layer "B.Cu") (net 25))
 (segment (start 125.095 96.52) (end 127 96.52) (width 1.5) (layer "B.Cu") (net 25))
 (segment (start 137.16 97.536) (end 132.588 97.536) (width 1.5) (layer "B.Cu") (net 25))
 (segment (start 146.685 55.245) (end 146.685 65.405) (width 1.5) (layer "F.Cu") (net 9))
 (via (at 146.685 65.405) (size 3) (drill 2) (layers "F.Cu" "B.Cu") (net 9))
 (via (at 146.685 55.245) (size 3) (drill 2) (layers "F.Cu" "B.Cu") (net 9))
 (segment (start 111.76 55.245) (end 146.685 55.245) (width 1.5) (layer "B.Cu") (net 9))
 (segment (start 99.695 67.31) (end 111.76 55.245) (width 1.5) (layer "B.Cu") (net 9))
 (segment (start 146.685 64.77) (end 146.685 84.455) (width 1.5) (layer "B.Cu") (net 9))
 (segment (start 100.965 101.6) (end 99.695 100.33) (width 1.5) (layer "B.Cu") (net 9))
 (segment (start 139.192 91.948) (end 137.16 93.98) (width 1.5) (layer "B.Cu") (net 9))
 (segment (start 137.16 93.98) (end 127 93.98) (width 1.5) (layer "B.Cu") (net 9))
 (segment (start 146.685 84.455) (end 139.192 91.948) (width 1.5) (layer "B.Cu") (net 9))
 (segment (start 103.45 101.6) (end 100.965 101.6) (width 1.5) (layer "B.Cu") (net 9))
 (segment (start 99.695 100.33) (end 99.695 67.31) (width 1.5) (layer "B.Cu") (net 9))
 (segment (start 125.715 83.2) (end 127 81.915) (width 1.5) (layer "B.Cu") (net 26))
 (segment (start 127 81.915) (end 127 79.76) (width 1.5) (layer "B.Cu") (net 26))
 (segment (start 121.92 83.2) (end 125.715 83.2) (width 1.5) (layer "B.Cu") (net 26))
 (segment (start 126.488 77.22) (end 127 77.22) (width 1.5) (layer "B.Cu") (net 27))
 (segment (start 121.92 80.66) (end 123.048 80.66) (width 1.5) (layer "B.Cu") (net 27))
 (segment (start 123.048 80.66) (end 126.488 77.22) (width 1.5) (layer "B.Cu") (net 27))
 (segment (start 125.984 74.676) (end 125.988 74.68) (width 1.5) (layer "B.Cu") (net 28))
 (segment (start 121.92 78.12) (end 122.54 78.12) (width 1.5) (layer "B.Cu") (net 28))
 (segment (start 125.988 74.68) (end 127 74.68) (width 1.5) (layer "B.Cu") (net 28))
 (segment (start 122.54 78.12) (end 125.984 74.676) (width 1.5) (layer "B.Cu") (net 28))
 (segment (start 123.332 70.5) (end 124.972 72.14) (width 1.5) (layer "B.Cu") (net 29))
 (segment (start 124.972 72.14) (end 127 72.14) (width 1.5) (layer "B.Cu") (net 29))
 (segment (start 121.92 70.5) (end 123.332 70.5) (width 1.5) (layer "B.Cu") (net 29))
 (segment (start 123.84 67.96) (end 125.48 69.6) (width 1.5) (layer "B.Cu") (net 30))
 (segment (start 125.48 69.6) (end 127 69.6) (width 1.5) (layer "B.Cu") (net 30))
 (segment (start 121.92 67.96) (end 123.84 67.96) (width 1.5) (layer "B.Cu") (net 30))
 (segment (start 118.685 98.76) (end 120.105 100.18) (width 2) (layer "B.Cu") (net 4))
 (segment (start 95.105 100.18) (end 95.105 92.855) (width 2) (layer "B.Cu") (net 4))
 (segment (start 119.38 71.628) (end 115.697 67.945) (width 2) (layer "B.Cu") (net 4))
 (segment (start 120.792 85.74) (end 120.635 85.74) (width 2) (layer "B.Cu") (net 4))
 (segment (start 120.635 85.74) (end 118.745 87.63) (width 2) (layer "B.Cu") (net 4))
 (segment (start 121.92 75.58) (end 121.92 73.04) (width 1.5) (layer "B.Cu") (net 4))
 (segment (start 112.268 67.945) (end 109.22 67.945) (width 2) (layer "B.Cu") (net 4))
 (segment (start 112.268 81.339081) (end 112.268 67.945) (width 2) (layer "B.Cu") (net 4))
 (segment (start 134.62 73.54863) (end 128.13137 67.06) (width 2) (layer "B.Cu") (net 4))
 (segment (start 120.792 73.04) (end 119.38 71.628) (width 2) (layer "B.Cu") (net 4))
 (segment (start 121.92 73.04) (end 120.792 73.04) (width 2) (layer "B.Cu") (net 4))
 (segment (start 120.792 85.74) (end 119.38 84.328) (width 2) (layer "B.Cu") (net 4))
 (segment (start 128.13137 67.06) (end 127 67.06) (width 2) (layer "B.Cu") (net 4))
 (segment (start 134.62 82.55) (end 134.62 73.54863) (width 2) (layer "B.Cu") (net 4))
 (segment (start 119.38 84.328) (end 119.38 71.628) (width 2) (layer "B.Cu") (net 4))
 (segment (start 117.14 98.76) (end 118.685 98.76) (width 2) (layer "B.Cu") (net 4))
 (segment (start 114.6 98.76) (end 114.3 98.76) (width 1.5) (layer "B.Cu") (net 4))
 (segment (start 110.422081 83.185) (end 112.268 81.339081) (width 2) (layer "B.Cu") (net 4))
 (segment (start 109.22 83.185) (end 110.422081 83.185) (width 2) (layer "B.Cu") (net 4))
 (segment (start 118.745 98.7) (end 118.685 98.76) (width 2) (layer "B.Cu") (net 4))
 (segment (start 113.145 98.76) (end 114.3 98.76) (width 1.5) (layer "B.Cu") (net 4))
 (segment (start 95.105 92.855) (end 97.155 90.805) (width 2) (layer "B.Cu") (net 4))
 (segment (start 115.697 67.945) (end 112.268 67.945) (width 2) (layer "B.Cu") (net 4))
 (segment (start 117.14 98.76) (end 113.145 98.76) (width 2) (layer "B.Cu") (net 4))
 (segment (start 118.745 87.63) (end 118.745 98.7) (width 2) (layer "B.Cu") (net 4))
 (segment (start 121.92 85.74) (end 120.792 85.74) (width 2) (layer "B.Cu") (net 4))
 (segment (start 121.92 85.74) (end 131.43 85.74) (width 2) (layer "B.Cu") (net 4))
 (segment (start 131.43 85.74) (end 134.62 82.55) (width 2) (layer "B.Cu") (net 4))
 (segment (start 104.775 73.025) (end 109.22 73.025) (width 2) (layer "B.Cu") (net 32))
 (segment (start 109.22 75.565) (end 104.775 75.565) (width 2) (layer "B.Cu") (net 33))
 (segment (start 104.775 78.105) (end 109.22 78.105) (width 2) (layer "B.Cu") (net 34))
 (segment (start 109.22 80.645) (end 104.775 80.645) (width 2) (layer "B.Cu") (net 35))
 (segment (start 107.605 98.76) (end 107.605 97.627) (width 1.5) (layer "B.Cu") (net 2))
 (segment (start 107.605 99.477) (end 107.605 98.76) (width 1.5) (layer "B.Cu") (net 2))
 (segment (start 107.605 97.627) (end 111.8235 93.4085) (width 1.5) (layer "B.Cu") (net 2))
 (segment (start 111.8235 93.4085) (end 112.395 93.98) (width 2) (layer "B.Cu") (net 2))
 (segment (start 109.22 90.805) (end 111.8235 93.4085) (width 2) (layer "B.Cu") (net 2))
 (segment (start 108.99 103.91) (end 108.99 101.6) (width 1.5) (layer "B.Cu") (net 2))
 (segment (start 104.655 90.805) (end 109.22 90.805) (width 2) (layer "B.Cu") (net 2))
 (segment (start 114.3 109.22) (end 108.99 103.91) (width 1.5) (layer "B.Cu") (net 2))
 (segment (start 108.99 101.6) (end 108.99 100.862) (width 1.5) (layer "B.Cu") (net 2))
 (segment (start 125.73 109.22) (end 114.3 109.22) (width 1.5) (layer "B.Cu") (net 2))
 (segment (start 108.99 100.862) (end 107.605 99.477) (width 1.5) (layer "B.Cu") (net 2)))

